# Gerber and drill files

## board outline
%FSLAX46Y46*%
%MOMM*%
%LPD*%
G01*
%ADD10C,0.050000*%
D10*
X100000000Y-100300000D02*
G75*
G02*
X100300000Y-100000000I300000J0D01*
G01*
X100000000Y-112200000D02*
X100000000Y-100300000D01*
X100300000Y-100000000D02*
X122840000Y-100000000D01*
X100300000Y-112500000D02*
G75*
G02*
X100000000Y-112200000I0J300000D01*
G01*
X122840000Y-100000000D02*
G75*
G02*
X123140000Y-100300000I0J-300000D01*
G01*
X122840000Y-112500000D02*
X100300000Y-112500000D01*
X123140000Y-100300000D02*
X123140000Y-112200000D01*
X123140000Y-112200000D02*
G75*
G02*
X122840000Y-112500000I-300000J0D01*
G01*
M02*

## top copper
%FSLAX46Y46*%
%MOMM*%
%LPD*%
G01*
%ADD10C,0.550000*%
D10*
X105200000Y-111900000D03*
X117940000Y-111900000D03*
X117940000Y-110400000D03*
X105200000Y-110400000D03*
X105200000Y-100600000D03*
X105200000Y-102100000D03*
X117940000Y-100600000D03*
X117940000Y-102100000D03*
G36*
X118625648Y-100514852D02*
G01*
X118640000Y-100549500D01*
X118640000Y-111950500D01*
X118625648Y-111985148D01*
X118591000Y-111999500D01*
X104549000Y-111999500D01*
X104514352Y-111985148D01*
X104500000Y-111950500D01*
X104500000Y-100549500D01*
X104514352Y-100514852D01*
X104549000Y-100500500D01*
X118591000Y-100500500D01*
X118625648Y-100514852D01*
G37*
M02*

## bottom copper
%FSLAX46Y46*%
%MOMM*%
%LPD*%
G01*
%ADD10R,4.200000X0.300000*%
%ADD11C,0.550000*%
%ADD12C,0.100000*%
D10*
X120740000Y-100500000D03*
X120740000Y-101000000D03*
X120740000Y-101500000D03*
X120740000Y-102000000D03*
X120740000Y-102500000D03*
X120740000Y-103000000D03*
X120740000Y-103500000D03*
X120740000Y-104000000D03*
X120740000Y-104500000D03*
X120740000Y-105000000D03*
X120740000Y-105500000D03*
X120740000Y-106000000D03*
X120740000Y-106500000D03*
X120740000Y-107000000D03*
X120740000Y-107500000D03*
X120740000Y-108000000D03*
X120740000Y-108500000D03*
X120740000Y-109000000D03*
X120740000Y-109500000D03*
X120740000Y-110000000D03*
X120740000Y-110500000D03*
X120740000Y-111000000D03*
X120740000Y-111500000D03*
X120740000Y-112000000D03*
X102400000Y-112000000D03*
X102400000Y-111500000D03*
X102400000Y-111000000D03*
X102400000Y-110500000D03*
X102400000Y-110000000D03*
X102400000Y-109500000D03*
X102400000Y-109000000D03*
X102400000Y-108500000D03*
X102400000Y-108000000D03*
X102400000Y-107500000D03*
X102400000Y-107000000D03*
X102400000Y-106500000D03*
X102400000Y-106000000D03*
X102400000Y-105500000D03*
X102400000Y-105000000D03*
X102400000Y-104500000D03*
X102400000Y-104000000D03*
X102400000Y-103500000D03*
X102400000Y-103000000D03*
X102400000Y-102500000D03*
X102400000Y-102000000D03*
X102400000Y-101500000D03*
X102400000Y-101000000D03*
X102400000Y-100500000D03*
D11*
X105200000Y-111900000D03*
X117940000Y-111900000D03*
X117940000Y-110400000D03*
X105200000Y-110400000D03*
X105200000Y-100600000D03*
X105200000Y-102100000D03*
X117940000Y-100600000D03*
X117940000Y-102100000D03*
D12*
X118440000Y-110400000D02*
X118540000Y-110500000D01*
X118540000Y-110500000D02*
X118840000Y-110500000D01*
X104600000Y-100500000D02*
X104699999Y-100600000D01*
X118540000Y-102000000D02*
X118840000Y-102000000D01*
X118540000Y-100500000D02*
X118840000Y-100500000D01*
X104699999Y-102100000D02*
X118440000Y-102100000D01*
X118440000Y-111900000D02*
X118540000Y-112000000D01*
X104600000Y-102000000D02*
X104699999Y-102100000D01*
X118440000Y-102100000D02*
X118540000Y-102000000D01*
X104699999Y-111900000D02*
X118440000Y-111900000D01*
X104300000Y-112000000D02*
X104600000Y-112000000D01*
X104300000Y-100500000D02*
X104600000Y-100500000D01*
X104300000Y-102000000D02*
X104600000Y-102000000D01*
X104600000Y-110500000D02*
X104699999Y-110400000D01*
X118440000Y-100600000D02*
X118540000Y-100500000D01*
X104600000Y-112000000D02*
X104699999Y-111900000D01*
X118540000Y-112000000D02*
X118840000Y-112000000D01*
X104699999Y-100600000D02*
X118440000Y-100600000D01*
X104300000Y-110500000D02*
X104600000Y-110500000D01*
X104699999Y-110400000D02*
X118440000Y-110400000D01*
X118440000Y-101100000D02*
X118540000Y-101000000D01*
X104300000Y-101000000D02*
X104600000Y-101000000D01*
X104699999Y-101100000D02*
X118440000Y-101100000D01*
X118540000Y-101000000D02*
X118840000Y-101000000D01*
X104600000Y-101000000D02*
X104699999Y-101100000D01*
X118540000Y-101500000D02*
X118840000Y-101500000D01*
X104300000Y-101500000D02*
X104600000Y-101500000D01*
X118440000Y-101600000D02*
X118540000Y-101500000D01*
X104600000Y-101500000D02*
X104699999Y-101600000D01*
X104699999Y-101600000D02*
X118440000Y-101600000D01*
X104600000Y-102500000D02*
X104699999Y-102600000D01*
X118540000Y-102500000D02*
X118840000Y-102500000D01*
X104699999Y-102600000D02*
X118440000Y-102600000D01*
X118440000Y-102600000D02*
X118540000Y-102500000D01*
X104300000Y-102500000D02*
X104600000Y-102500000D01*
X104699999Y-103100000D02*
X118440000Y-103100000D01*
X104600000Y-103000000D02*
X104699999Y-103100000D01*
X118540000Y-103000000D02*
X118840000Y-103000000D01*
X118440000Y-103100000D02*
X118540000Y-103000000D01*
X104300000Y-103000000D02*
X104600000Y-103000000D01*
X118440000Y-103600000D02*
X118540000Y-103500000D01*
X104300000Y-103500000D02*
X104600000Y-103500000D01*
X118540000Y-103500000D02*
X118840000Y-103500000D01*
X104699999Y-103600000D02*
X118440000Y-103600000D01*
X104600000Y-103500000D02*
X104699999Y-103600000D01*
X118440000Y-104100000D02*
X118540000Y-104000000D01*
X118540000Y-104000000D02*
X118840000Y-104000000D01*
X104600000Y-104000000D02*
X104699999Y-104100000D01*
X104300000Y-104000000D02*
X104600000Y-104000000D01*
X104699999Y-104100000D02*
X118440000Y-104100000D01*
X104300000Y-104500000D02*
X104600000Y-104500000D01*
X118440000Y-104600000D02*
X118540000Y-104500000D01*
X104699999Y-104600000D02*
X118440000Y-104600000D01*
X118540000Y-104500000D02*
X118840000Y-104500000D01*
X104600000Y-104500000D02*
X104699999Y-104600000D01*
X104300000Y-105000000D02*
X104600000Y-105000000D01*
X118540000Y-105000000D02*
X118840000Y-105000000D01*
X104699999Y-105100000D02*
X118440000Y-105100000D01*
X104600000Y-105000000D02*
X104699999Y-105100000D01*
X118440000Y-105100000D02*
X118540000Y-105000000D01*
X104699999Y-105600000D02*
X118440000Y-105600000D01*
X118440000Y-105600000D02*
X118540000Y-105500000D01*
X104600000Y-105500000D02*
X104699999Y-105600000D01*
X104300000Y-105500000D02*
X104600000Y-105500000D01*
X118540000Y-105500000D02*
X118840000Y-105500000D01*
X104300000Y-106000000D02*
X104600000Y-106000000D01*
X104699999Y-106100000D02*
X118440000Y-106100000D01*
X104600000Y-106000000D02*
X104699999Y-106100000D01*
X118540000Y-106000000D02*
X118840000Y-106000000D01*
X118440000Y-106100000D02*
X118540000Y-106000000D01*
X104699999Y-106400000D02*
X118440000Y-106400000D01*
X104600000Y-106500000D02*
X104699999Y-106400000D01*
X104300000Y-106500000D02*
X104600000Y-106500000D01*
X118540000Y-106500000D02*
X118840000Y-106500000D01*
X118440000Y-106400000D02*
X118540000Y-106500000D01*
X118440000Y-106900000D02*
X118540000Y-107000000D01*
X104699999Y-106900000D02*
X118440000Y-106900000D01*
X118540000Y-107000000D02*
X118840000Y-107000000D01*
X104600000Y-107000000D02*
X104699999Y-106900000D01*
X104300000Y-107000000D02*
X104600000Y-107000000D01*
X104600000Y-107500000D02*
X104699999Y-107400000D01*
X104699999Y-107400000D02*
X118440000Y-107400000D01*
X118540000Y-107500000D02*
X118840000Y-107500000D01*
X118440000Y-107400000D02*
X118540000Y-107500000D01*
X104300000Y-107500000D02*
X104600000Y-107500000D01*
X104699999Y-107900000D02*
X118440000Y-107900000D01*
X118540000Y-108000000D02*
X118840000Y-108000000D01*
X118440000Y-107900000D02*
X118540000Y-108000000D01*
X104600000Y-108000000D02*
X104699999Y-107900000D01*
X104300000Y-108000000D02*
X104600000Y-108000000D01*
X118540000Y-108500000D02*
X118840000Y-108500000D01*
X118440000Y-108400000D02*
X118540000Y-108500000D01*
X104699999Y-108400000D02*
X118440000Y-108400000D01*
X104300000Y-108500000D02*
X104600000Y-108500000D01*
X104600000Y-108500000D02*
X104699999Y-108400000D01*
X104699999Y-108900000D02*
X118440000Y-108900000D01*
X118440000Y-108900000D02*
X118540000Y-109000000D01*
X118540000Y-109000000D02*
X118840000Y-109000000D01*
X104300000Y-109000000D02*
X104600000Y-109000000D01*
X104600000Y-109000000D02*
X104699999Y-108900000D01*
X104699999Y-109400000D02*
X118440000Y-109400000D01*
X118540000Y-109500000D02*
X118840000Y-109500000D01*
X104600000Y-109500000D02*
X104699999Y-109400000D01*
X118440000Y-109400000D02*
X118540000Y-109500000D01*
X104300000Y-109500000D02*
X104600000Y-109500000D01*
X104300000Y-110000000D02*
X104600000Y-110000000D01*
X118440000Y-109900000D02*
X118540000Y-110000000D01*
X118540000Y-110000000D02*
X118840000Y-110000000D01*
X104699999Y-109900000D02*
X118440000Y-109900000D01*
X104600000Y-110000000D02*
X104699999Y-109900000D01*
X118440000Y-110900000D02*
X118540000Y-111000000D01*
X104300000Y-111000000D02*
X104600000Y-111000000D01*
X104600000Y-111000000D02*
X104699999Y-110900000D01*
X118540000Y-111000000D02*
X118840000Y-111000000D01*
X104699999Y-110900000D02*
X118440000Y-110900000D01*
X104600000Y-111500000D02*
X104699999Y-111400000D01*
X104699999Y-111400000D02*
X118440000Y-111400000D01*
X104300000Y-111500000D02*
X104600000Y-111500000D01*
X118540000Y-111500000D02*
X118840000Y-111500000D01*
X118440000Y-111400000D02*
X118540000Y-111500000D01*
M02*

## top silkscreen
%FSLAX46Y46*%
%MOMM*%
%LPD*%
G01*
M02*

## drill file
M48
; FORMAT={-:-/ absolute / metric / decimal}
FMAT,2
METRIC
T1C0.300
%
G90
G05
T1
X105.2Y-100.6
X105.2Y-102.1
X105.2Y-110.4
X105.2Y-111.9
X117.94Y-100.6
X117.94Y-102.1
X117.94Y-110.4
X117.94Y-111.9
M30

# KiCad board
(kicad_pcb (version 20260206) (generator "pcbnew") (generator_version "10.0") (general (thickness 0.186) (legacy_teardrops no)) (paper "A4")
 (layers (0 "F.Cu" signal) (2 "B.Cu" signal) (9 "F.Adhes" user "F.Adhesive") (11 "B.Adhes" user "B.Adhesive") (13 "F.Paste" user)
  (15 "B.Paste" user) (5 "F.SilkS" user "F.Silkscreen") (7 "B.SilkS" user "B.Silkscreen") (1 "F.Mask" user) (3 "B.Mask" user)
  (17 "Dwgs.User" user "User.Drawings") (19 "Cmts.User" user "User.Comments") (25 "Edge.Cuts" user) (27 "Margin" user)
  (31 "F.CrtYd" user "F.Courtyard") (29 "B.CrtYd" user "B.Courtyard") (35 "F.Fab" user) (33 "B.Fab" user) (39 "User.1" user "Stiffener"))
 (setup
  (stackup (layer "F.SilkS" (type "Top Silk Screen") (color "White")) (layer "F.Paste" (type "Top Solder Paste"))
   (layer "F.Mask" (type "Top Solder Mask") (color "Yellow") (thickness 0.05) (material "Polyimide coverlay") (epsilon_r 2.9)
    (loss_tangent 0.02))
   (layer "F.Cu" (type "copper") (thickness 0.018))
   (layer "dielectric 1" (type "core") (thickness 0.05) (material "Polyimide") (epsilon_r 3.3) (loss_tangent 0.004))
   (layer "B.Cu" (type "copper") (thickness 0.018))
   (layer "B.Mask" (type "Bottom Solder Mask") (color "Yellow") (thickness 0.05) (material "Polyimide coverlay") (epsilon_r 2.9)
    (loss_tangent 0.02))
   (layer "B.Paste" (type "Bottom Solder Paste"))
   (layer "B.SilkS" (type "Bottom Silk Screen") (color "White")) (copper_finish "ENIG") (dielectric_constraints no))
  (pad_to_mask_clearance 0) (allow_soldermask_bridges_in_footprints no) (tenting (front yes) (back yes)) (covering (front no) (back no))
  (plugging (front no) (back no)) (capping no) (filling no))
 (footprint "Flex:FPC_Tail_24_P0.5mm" (layer "B.Cu") (at 123.14 106.25 90)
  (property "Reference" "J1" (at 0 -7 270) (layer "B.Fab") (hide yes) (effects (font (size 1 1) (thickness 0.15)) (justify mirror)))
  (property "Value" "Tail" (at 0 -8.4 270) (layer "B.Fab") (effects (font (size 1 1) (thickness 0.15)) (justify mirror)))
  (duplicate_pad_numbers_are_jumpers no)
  (pad "1" smd rect (at 5.75 -2.4 90) (size 0.3 4.2) (layers "B.Cu") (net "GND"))
  (pad "2" smd rect (at 5.25 -2.4 90) (size 0.3 4.2) (layers "B.Cu") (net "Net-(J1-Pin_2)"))
  (pad "3" smd rect (at 4.75 -2.4 90) (size 0.3 4.2) (layers "B.Cu") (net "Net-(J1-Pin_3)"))
  (pad "4" smd rect (at 4.25 -2.4 90) (size 0.3 4.2) (layers "B.Cu") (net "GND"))
  (pad "5" smd rect (at 3.75 -2.4 90) (size 0.3 4.2) (layers "B.Cu") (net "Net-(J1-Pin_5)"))
  (pad "6" smd rect (at 3.25 -2.4 90) (size 0.3 4.2) (layers "B.Cu") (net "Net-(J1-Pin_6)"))
  (pad "7" smd rect (at 2.75 -2.4 90) (size 0.3 4.2) (layers "B.Cu") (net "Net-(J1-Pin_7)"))
  (pad "8" smd rect (at 2.25 -2.4 90) (size 0.3 4.2) (layers "B.Cu") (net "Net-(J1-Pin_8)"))
  (pad "9" smd rect (at 1.75 -2.4 90) (size 0.3 4.2) (layers "B.Cu") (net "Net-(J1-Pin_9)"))
  (pad "10" smd rect (at 1.25 -2.4 90) (size 0.3 4.2) (layers "B.Cu") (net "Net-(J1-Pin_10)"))
  (pad "11" smd rect (at 0.75 -2.4 90) (size 0.3 4.2) (layers "B.Cu") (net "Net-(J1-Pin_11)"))
  (pad "12" smd rect (at 0.25 -2.4 90) (size 0.3 4.2) (layers "B.Cu") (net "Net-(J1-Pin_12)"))
  (pad "13" smd rect (at -0.25 -2.4 90) (size 0.3 4.2) (layers "B.Cu") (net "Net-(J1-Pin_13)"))
  (pad "14" smd rect (at -0.75 -2.4 90) (size 0.3 4.2) (layers "B.Cu") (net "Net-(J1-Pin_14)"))
  (pad "15" smd rect (at -1.25 -2.4 90) (size 0.3 4.2) (layers "B.Cu") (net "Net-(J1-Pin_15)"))
  (pad "16" smd rect (at -1.75 -2.4 90) (size 0.3 4.2) (layers "B.Cu") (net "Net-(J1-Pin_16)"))
  (pad "17" smd rect (at -2.25 -2.4 90) (size 0.3 4.2) (layers "B.Cu") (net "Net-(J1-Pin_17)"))
  (pad "18" smd rect (at -2.75 -2.4 90) (size 0.3 4.2) (layers "B.Cu") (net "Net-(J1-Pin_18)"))
  (pad "19" smd rect (at -3.25 -2.4 90) (size 0.3 4.2) (layers "B.Cu") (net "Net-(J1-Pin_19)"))
  (pad "20" smd rect (at -3.75 -2.4 90) (size 0.3 4.2) (layers "B.Cu") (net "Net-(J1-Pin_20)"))
  (pad "21" smd rect (at -4.25 -2.4 90) (size 0.3 4.2) (layers "B.Cu") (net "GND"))
  (pad "22" smd rect (at -4.75 -2.4 90) (size 0.3 4.2) (layers "B.Cu") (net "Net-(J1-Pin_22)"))
  (pad "23" smd rect (at -5.25 -2.4 90) (size 0.3 4.2) (layers "B.Cu") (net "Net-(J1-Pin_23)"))
  (pad "24" smd rect (at -5.75 -2.4 90) (size 0.3 4.2) (layers "B.Cu") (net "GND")))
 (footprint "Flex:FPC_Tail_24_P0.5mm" (layer "B.Cu") (at 100 106.25 -90)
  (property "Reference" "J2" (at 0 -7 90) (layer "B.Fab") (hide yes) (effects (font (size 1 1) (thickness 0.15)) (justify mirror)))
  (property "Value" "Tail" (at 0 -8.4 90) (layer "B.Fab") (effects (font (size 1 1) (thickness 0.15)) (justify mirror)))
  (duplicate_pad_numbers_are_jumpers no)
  (pad "1" smd rect (at 5.75 -2.4 270) (size 0.3 4.2) (layers "B.Cu") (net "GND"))
  (pad "2" smd rect (at 5.25 -2.4 270) (size 0.3 4.2) (layers "B.Cu") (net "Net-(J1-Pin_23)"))
  (pad "3" smd rect (at 4.75 -2.4 270) (size 0.3 4.2) (layers "B.Cu") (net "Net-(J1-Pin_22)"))
  (pad "4" smd rect (at 4.25 -2.4 270) (size 0.3 4.2) (layers "B.Cu") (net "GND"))
  (pad "5" smd rect (at 3.75 -2.4 270) (size 0.3 4.2) (layers "B.Cu") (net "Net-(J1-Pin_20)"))
  (pad "6" smd rect (at 3.25 -2.4 270) (size 0.3 4.2) (layers "B.Cu") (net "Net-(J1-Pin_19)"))
  (pad "7" smd rect (at 2.75 -2.4 270) (size 0.3 4.2) (layers "B.Cu") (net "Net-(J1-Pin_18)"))
  (pad "8" smd rect (at 2.25 -2.4 270) (size 0.3 4.2) (layers "B.Cu") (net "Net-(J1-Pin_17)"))
  (pad "9" smd rect (at 1.75 -2.4 270) (size 0.3 4.2) (layers "B.Cu") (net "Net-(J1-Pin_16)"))
  (pad "10" smd rect (at 1.25 -2.4 270) (size 0.3 4.2) (layers "B.Cu") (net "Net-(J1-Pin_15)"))
  (pad "11" smd rect (at 0.75 -2.4 270) (size 0.3 4.2) (layers "B.Cu") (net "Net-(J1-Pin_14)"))
  (pad "12" smd rect (at 0.25 -2.4 270) (size 0.3 4.2) (layers "B.Cu") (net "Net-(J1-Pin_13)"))
  (pad "13" smd rect (at -0.25 -2.4 270) (size 0.3 4.2) (layers "B.Cu") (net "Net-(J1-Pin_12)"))
  (pad "14" smd rect (at -0.75 -2.4 270) (size 0.3 4.2) (layers "B.Cu") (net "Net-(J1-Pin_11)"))
  (pad "15" smd rect (at -1.25 -2.4 270) (size 0.3 4.2) (layers "B.Cu") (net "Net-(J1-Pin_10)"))
  (pad "16" smd rect (at -1.75 -2.4 270) (size 0.3 4.2) (layers "B.Cu") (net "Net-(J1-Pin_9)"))
  (pad "17" smd rect (at -2.25 -2.4 270) (size 0.3 4.2) (layers "B.Cu") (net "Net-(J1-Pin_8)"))
  (pad "18" smd rect (at -2.75 -2.4 270) (size 0.3 4.2) (layers "B.Cu") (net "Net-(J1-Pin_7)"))
  (pad "19" smd rect (at -3.25 -2.4 270) (size 0.3 4.2) (layers "B.Cu") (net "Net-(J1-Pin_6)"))
  (pad "20" smd rect (at -3.75 -2.4 270) (size 0.3 4.2) (layers "B.Cu") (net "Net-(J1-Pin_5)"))
  (pad "21" smd rect (at -4.25 -2.4 270) (size 0.3 4.2) (layers "B.Cu") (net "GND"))
  (pad "22" smd rect (at -4.75 -2.4 270) (size 0.3 4.2) (layers "B.Cu") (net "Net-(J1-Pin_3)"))
  (pad "23" smd rect (at -5.25 -2.4 270) (size 0.3 4.2) (layers "B.Cu") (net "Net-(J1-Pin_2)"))
  (pad "24" smd rect (at -5.75 -2.4 270) (size 0.3 4.2) (layers "B.Cu") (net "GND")))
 (gr_arc (start 100 100.3) (mid 100.087867 100.087867) (end 100.3 100) (stroke (width 0.05) (type default)) (layer "Edge.Cuts"))
 (gr_line (start 100 112.2) (end 100 100.3) (stroke (width 0.05) (type default)) (layer "Edge.Cuts"))
 (gr_line (start 100.3 100) (end 122.84 100) (stroke (width 0.05) (type default)) (layer "Edge.Cuts"))
 (gr_arc (start 100.3 112.5) (mid 100.087867 112.412132) (end 100 112.2) (stroke (width 0.05) (type default)) (layer "Edge.Cuts"))
 (gr_arc (start 122.84 100) (mid 123.052132 100.087867) (end 123.14 100.3) (stroke (width 0.05) (type default)) (layer "Edge.Cuts"))
 (gr_line (start 122.84 112.5) (end 100.3 112.5) (stroke (width 0.05) (type default)) (layer "Edge.Cuts"))
 (gr_line (start 123.14 100.3) (end 123.14 112.2) (stroke (width 0.05) (type default)) (layer "Edge.Cuts"))
 (gr_arc (start 123.14 112.2) (mid 123.052132 112.412132) (end 122.84 112.5) (stroke (width 0.05) (type default)) (layer "Edge.Cuts"))
 (via (at 105.2 111.9) (size 0.55) (drill 0.3) (layers "F.Cu" "B.Cu") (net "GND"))
 (via (at 117.94 111.9) (size 0.55) (drill 0.3) (layers "F.Cu" "B.Cu") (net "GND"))
 (via (at 117.94 110.4) (size 0.55) (drill 0.3) (layers "F.Cu" "B.Cu") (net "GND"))
 (via (at 105.2 110.4) (size 0.55) (drill 0.3) (layers "F.Cu" "B.Cu") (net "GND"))
 (via (at 105.2 100.6) (size 0.55) (drill 0.3) (layers "F.Cu" "B.Cu") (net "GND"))
 (via (at 105.2 102.1) (size 0.55) (drill 0.3) (layers "F.Cu" "B.Cu") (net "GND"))
 (via (at 117.94 100.6) (size 0.55) (drill 0.3) (layers "F.Cu" "B.Cu") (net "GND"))
 (via (at 117.94 102.1) (size 0.55) (drill 0.3) (layers "F.Cu" "B.Cu") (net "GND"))
 (segment (start 118.44 110.4) (end 118.54 110.5) (width 0.1) (layer "B.Cu") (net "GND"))
 (segment (start 118.54 110.5) (end 118.84 110.5) (width 0.1) (layer "B.Cu") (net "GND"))
 (segment (start 104.6 100.5) (end 104.699999 100.6) (width 0.1) (layer "B.Cu") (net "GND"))
 (segment (start 118.54 102) (end 118.84 102) (width 0.1) (layer "B.Cu") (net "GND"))
 (segment (start 118.54 100.5) (end 118.84 100.5) (width 0.1) (layer "B.Cu") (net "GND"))
 (segment (start 104.699999 102.1) (end 118.44 102.1) (width 0.1) (layer "B.Cu") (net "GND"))
 (segment (start 118.44 111.9) (end 118.54 112) (width 0.1) (layer "B.Cu") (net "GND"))
 (segment (start 104.6 102) (end 104.699999 102.1) (width 0.1) (layer "B.Cu") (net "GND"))
 (segment (start 118.44 102.1) (end 118.54 102) (width 0.1) (layer "B.Cu") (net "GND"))
 (segment (start 104.699999 111.9) (end 118.44 111.9) (width 0.1) (layer "B.Cu") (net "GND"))
 (segment (start 104.3 112) (end 104.6 112) (width 0.1) (layer "B.Cu") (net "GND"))
 (segment (start 104.3 100.5) (end 104.6 100.5) (width 0.1) (layer "B.Cu") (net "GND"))
 (segment (start 104.3 102) (end 104.6 102) (width 0.1) (layer "B.Cu") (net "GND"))
 (segment (start 104.6 110.5) (end 104.699999 110.4) (width 0.1) (layer "B.Cu") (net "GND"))
 (segment (start 118.44 100.6) (end 118.54 100.5) (width 0.1) (layer "B.Cu") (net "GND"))
 (segment (start 104.6 112) (end 104.699999 111.9) (width 0.1) (layer "B.Cu") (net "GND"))
 (segment (start 118.54 112) (end 118.84 112) (width 0.1) (layer "B.Cu") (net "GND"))
 (segment (start 104.699999 100.6) (end 118.44 100.6) (width 0.1) (layer "B.Cu") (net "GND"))
 (segment (start 104.3 110.5) (end 104.6 110.5) (width 0.1) (layer "B.Cu") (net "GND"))
 (segment (start 104.699999 110.4) (end 118.44 110.4) (width 0.1) (layer "B.Cu") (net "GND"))
 (segment (start 118.44 101.1) (end 118.54 101) (width 0.1) (layer "B.Cu") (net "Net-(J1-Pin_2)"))
 (segment (start 104.3 101) (end 104.6 101) (width 0.1) (layer "B.Cu") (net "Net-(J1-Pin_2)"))
 (segment (start 104.699999 101.1) (end 118.44 101.1) (width 0.1) (layer "B.Cu") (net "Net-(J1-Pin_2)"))
 (segment (start 118.54 101) (end 118.84 101) (width 0.1) (layer "B.Cu") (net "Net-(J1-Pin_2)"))
 (segment (start 104.6 101) (end 104.699999 101.1) (width 0.1) (layer "B.Cu") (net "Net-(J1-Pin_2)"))
 (segment (start 118.54 101.5) (end 118.84 101.5) (width 0.1) (layer "B.Cu") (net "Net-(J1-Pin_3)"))
 (segment (start 104.3 101.5) (end 104.6 101.5) (width 0.1) (layer "B.Cu") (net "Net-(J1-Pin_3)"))
 (segment (start 118.44 101.6) (end 118.54 101.5) (width 0.1) (layer "B.Cu") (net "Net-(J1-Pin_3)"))
 (segment (start 104.6 101.5) (end 104.699999 101.6) (width 0.1) (layer "B.Cu") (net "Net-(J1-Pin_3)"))
 (segment (start 104.699999 101.6) (end 118.44 101.6) (width 0.1) (layer "B.Cu") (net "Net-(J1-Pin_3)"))
 (segment (start 104.6 102.5) (end 104.699999 102.6) (width 0.1) (layer "B.Cu") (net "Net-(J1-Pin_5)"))
 (segment (start 118.54 102.5) (end 118.84 102.5) (width 0.1) (layer "B.Cu") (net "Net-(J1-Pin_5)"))
 (segment (start 104.699999 102.6) (end 118.44 102.6) (width 0.1) (layer "B.Cu") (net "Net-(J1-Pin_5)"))
 (segment (start 118.44 102.6) (end 118.54 102.5) (width 0.1) (layer "B.Cu") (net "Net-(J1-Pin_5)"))
 (segment (start 104.3 102.5) (end 104.6 102.5) (width 0.1) (layer "B.Cu") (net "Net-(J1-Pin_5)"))
 (segment (start 104.699999 103.1) (end 118.44 103.1) (width 0.1) (layer "B.Cu") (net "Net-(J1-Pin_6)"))
 (segment (start 104.6 103) (end 104.699999 103.1) (width 0.1) (layer "B.Cu") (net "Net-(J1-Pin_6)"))
 (segment (start 118.54 103) (end 118.84 103) (width 0.1) (layer "B.Cu") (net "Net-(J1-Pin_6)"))
 (segment (start 118.44 103.1) (end 118.54 103) (width 0.1) (layer "B.Cu") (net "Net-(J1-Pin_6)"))
 (segment (start 104.3 103) (end 104.6 103) (width 0.1) (layer "B.Cu") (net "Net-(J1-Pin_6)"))
 (segment (start 118.44 103.6) (end 118.54 103.5) (width 0.1) (layer "B.Cu") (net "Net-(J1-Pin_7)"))
 (segment (start 104.3 103.5) (end 104.6 103.5) (width 0.1) (layer "B.Cu") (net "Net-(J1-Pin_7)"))
 (segment (start 118.54 103.5) (end 118.84 103.5) (width 0.1) (layer "B.Cu") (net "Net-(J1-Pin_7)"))
 (segment (start 104.699999 103.6) (end 118.44 103.6) (width 0.1) (layer "B.Cu") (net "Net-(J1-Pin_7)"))
 (segment (start 104.6 103.5) (end 104.699999 103.6) (width 0.1) (layer "B.Cu") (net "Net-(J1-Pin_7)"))
 (segment (start 118.44 104.1) (end 118.54 104) (width 0.1) (layer "B.Cu") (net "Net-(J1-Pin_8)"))
 (segment (start 118.54 104) (end 118.84 104) (width 0.1) (layer "B.Cu") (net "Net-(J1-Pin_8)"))
 (segment (start 104.6 104) (end 104.699999 104.1) (width 0.1) (layer "B.Cu") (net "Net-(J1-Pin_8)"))
 (segment (start 104.3 104) (end 104.6 104) (width 0.1) (layer "B.Cu") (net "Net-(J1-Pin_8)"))
 (segment (start 104.699999 104.1) (end 118.44 104.1) (width 0.1) (layer "B.Cu") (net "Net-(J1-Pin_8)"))
 (segment (start 104.3 104.5) (end 104.6 104.5) (width 0.1) (layer "B.Cu") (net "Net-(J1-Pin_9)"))
 (segment (start 118.44 104.6) (end 118.54 104.5) (width 0.1) (layer "B.Cu") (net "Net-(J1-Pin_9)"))
 (segment (start 104.699999 104.6) (end 118.44 104.6) (width 0.1) (layer "B.Cu") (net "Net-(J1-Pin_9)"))
 (segment (start 118.54 104.5) (end 118.84 104.5) (width 0.1) (layer "B.Cu") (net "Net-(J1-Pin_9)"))
 (segment (start 104.6 104.5) (end 104.699999 104.6) (width 0.1) (layer "B.Cu") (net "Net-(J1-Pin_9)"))
 (segment (start 104.3 105) (end 104.6 105) (width 0.1) (layer "B.Cu") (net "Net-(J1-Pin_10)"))
 (segment (start 118.54 105) (end 118.84 105) (width 0.1) (layer "B.Cu") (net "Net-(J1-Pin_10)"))
 (segment (start 104.699999 105.1) (end 118.44 105.1) (width 0.1) (layer "B.Cu") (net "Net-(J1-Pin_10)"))
 (segment (start 104.6 105) (end 104.699999 105.1) (width 0.1) (layer "B.Cu") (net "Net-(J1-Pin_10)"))
 (segment (start 118.44 105.1) (end 118.54 105) (width 0.1) (layer "B.Cu") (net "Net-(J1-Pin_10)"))
 (segment (start 104.699999 105.6) (end 118.44 105.6) (width 0.1) (layer "B.Cu") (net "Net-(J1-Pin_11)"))
 (segment (start 118.44 105.6) (end 118.54 105.5) (width 0.1) (layer "B.Cu") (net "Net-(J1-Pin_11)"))
 (segment (start 104.6 105.5) (end 104.699999 105.6) (width 0.1) (layer "B.Cu") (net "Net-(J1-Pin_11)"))
 (segment (start 104.3 105.5) (end 104.6 105.5) (width 0.1) (layer "B.Cu") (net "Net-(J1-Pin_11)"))
 (segment (start 118.54 105.5) (end 118.84 105.5) (width 0.1) (layer "B.Cu") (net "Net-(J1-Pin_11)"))
 (segment (start 104.3 106) (end 104.6 106) (width 0.1) (layer "B.Cu") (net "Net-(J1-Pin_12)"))
 (segment (start 104.699999 106.1) (end 118.44 106.1) (width 0.1) (layer "B.Cu") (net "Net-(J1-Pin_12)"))
 (segment (start 104.6 106) (end 104.699999 106.1) (width 0.1) (layer "B.Cu") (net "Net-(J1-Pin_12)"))
 (segment (start 118.54 106) (end 118.84 106) (width 0.1) (layer "B.Cu") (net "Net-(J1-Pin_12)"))
 (segment (start 118.44 106.1) (end 118.54 106) (width 0.1) (layer "B.Cu") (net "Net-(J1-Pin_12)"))
 (segment (start 104.699999 106.4) (end 118.44 106.4) (width 0.1) (layer "B.Cu") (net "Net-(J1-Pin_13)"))
 (segment (start 104.6 106.5) (end 104.699999 106.4) (width 0.1) (layer "B.Cu") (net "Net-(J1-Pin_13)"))
 (segment (start 104.3 106.5) (end 104.6 106.5) (width 0.1) (layer "B.Cu") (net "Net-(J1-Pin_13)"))
 (segment (start 118.54 106.5) (end 118.84 106.5) (width 0.1) (layer "B.Cu") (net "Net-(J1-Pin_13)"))
 (segment (start 118.44 106.4) (end 118.54 106.5) (width 0.1) (layer "B.Cu") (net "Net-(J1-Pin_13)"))
 (segment (start 118.44 106.9) (end 118.54 107) (width 0.1) (layer "B.Cu") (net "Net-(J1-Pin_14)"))
 (segment (start 104.699999 106.9) (end 118.44 106.9) (width 0.1) (layer "B.Cu") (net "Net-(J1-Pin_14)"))
 (segment (start 118.54 107) (end 118.84 107) (width 0.1) (layer "B.Cu") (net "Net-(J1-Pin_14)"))
 (segment (start 104.6 107) (end 104.699999 106.9) (width 0.1) (layer "B.Cu") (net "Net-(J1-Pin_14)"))
 (segment (start 104.3 107) (end 104.6 107) (width 0.1) (layer "B.Cu") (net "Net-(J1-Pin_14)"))
 (segment (start 104.6 107.5) (end 104.699999 107.4) (width 0.1) (layer "B.Cu") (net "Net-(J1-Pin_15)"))
 (segment (start 104.699999 107.4) (end 118.44 107.4) (width 0.1) (layer "B.Cu") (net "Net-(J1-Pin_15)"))
 (segment (start 118.54 107.5) (end 118.84 107.5) (width 0.1) (layer "B.Cu") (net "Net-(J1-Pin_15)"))
 (segment (start 118.44 107.4) (end 118.54 107.5) (width 0.1) (layer "B.Cu") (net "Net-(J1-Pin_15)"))
 (segment (start 104.3 107.5) (end 104.6 107.5) (width 0.1) (layer "B.Cu") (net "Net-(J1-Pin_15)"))
 (segment (start 104.699999 107.9) (end 118.44 107.9) (width 0.1) (layer "B.Cu") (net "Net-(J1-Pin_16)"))
 (segment (start 118.54 108) (end 118.84 108) (width 0.1) (layer "B.Cu") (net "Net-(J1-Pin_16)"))
 (segment (start 118.44 107.9) (end 118.54 108) (width 0.1) (layer "B.Cu") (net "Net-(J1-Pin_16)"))
 (segment (start 104.6 108) (end 104.699999 107.9) (width 0.1) (layer "B.Cu") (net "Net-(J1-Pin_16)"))
 (segment (start 104.3 108) (end 104.6 108) (width 0.1) (layer "B.Cu") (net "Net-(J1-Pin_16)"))
 (segment (start 118.54 108.5) (end 118.84 108.5) (width 0.1) (layer "B.Cu") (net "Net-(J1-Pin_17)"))
 (segment (start 118.44 108.4) (end 118.54 108.5) (width 0.1) (layer "B.Cu") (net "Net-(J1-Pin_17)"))
 (segment (start 104.699999 108.4) (end 118.44 108.4) (width 0.1) (layer "B.Cu") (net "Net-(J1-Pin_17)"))
 (segment (start 104.3 108.5) (end 104.6 108.5) (width 0.1) (layer "B.Cu") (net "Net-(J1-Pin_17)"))
 (segment (start 104.6 108.5) (end 104.699999 108.4) (width 0.1) (layer "B.Cu") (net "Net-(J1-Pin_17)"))
 (segment (start 104.699999 108.9) (end 118.44 108.9) (width 0.1) (layer "B.Cu") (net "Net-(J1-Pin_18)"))
 (segment (start 118.44 108.9) (end 118.54 109) (width 0.1) (layer "B.Cu") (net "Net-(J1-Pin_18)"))
 (segment (start 118.54 109) (end 118.84 109) (width 0.1) (layer "B.Cu") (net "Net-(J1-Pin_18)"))
 (segment (start 104.3 109) (end 104.6 109) (width 0.1) (layer "B.Cu") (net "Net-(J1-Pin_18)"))
 (segment (start 104.6 109) (end 104.699999 108.9) (width 0.1) (layer "B.Cu") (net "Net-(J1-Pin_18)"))
 (segment (start 104.699999 109.4) (end 118.44 109.4) (width 0.1) (layer "B.Cu") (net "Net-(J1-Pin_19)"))
 (segment (start 118.54 109.5) (end 118.84 109.5) (width 0.1) (layer "B.Cu") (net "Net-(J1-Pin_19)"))
 (segment (start 104.6 109.5) (end 104.699999 109.4) (width 0.1) (layer "B.Cu") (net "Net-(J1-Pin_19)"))
 (segment (start 118.44 109.4) (end 118.54 109.5) (width 0.1) (layer "B.Cu") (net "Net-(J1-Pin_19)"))
 (segment (start 104.3 109.5) (end 104.6 109.5) (width 0.1) (layer "B.Cu") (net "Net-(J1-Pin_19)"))
 (segment (start 104.3 110) (end 104.6 110) (width 0.1) (layer "B.Cu") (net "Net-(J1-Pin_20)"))
 (segment (start 118.44 109.9) (end 118.54 110) (width 0.1) (layer "B.Cu") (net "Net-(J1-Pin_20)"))
 (segment (start 118.54 110) (end 118.84 110) (width 0.1) (layer "B.Cu") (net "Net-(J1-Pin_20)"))
 (segment (start 104.699999 109.9) (end 118.44 109.9) (width 0.1) (layer "B.Cu") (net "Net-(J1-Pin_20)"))
 (segment (start 104.6 110) (end 104.699999 109.9) (width 0.1) (layer "B.Cu") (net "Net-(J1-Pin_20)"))
 (segment (start 118.44 110.9) (end 118.54 111) (width 0.1) (layer "B.Cu") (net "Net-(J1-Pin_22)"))
 (segment (start 104.3 111) (end 104.6 111) (width 0.1) (layer "B.Cu") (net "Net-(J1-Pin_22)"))
 (segment (start 104.6 111) (end 104.699999 110.9) (width 0.1) (layer "B.Cu") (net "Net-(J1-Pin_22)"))
 (segment (start 118.54 111) (end 118.84 111) (width 0.1) (layer "B.Cu") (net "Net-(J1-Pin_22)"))
 (segment (start 104.699999 110.9) (end 118.44 110.9) (width 0.1) (layer "B.Cu") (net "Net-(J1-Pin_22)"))
 (segment (start 104.6 111.5) (end 104.699999 111.4) (width 0.1) (layer "B.Cu") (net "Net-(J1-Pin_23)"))
 (segment (start 104.699999 111.4) (end 118.44 111.4) (width 0.1) (layer "B.Cu") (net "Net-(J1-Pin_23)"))
 (segment (start 104.3 111.5) (end 104.6 111.5) (width 0.1) (layer "B.Cu") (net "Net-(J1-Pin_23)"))
 (segment (start 118.54 111.5) (end 118.84 111.5) (width 0.1) (layer "B.Cu") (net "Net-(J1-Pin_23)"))
 (segment (start 118.44 111.4) (end 118.54 111.5) (width 0.1) (layer "B.Cu") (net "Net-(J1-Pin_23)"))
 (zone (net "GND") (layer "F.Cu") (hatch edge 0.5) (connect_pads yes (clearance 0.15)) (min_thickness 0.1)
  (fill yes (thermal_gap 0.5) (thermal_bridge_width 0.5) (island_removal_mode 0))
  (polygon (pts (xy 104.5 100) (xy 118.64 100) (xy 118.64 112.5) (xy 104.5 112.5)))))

